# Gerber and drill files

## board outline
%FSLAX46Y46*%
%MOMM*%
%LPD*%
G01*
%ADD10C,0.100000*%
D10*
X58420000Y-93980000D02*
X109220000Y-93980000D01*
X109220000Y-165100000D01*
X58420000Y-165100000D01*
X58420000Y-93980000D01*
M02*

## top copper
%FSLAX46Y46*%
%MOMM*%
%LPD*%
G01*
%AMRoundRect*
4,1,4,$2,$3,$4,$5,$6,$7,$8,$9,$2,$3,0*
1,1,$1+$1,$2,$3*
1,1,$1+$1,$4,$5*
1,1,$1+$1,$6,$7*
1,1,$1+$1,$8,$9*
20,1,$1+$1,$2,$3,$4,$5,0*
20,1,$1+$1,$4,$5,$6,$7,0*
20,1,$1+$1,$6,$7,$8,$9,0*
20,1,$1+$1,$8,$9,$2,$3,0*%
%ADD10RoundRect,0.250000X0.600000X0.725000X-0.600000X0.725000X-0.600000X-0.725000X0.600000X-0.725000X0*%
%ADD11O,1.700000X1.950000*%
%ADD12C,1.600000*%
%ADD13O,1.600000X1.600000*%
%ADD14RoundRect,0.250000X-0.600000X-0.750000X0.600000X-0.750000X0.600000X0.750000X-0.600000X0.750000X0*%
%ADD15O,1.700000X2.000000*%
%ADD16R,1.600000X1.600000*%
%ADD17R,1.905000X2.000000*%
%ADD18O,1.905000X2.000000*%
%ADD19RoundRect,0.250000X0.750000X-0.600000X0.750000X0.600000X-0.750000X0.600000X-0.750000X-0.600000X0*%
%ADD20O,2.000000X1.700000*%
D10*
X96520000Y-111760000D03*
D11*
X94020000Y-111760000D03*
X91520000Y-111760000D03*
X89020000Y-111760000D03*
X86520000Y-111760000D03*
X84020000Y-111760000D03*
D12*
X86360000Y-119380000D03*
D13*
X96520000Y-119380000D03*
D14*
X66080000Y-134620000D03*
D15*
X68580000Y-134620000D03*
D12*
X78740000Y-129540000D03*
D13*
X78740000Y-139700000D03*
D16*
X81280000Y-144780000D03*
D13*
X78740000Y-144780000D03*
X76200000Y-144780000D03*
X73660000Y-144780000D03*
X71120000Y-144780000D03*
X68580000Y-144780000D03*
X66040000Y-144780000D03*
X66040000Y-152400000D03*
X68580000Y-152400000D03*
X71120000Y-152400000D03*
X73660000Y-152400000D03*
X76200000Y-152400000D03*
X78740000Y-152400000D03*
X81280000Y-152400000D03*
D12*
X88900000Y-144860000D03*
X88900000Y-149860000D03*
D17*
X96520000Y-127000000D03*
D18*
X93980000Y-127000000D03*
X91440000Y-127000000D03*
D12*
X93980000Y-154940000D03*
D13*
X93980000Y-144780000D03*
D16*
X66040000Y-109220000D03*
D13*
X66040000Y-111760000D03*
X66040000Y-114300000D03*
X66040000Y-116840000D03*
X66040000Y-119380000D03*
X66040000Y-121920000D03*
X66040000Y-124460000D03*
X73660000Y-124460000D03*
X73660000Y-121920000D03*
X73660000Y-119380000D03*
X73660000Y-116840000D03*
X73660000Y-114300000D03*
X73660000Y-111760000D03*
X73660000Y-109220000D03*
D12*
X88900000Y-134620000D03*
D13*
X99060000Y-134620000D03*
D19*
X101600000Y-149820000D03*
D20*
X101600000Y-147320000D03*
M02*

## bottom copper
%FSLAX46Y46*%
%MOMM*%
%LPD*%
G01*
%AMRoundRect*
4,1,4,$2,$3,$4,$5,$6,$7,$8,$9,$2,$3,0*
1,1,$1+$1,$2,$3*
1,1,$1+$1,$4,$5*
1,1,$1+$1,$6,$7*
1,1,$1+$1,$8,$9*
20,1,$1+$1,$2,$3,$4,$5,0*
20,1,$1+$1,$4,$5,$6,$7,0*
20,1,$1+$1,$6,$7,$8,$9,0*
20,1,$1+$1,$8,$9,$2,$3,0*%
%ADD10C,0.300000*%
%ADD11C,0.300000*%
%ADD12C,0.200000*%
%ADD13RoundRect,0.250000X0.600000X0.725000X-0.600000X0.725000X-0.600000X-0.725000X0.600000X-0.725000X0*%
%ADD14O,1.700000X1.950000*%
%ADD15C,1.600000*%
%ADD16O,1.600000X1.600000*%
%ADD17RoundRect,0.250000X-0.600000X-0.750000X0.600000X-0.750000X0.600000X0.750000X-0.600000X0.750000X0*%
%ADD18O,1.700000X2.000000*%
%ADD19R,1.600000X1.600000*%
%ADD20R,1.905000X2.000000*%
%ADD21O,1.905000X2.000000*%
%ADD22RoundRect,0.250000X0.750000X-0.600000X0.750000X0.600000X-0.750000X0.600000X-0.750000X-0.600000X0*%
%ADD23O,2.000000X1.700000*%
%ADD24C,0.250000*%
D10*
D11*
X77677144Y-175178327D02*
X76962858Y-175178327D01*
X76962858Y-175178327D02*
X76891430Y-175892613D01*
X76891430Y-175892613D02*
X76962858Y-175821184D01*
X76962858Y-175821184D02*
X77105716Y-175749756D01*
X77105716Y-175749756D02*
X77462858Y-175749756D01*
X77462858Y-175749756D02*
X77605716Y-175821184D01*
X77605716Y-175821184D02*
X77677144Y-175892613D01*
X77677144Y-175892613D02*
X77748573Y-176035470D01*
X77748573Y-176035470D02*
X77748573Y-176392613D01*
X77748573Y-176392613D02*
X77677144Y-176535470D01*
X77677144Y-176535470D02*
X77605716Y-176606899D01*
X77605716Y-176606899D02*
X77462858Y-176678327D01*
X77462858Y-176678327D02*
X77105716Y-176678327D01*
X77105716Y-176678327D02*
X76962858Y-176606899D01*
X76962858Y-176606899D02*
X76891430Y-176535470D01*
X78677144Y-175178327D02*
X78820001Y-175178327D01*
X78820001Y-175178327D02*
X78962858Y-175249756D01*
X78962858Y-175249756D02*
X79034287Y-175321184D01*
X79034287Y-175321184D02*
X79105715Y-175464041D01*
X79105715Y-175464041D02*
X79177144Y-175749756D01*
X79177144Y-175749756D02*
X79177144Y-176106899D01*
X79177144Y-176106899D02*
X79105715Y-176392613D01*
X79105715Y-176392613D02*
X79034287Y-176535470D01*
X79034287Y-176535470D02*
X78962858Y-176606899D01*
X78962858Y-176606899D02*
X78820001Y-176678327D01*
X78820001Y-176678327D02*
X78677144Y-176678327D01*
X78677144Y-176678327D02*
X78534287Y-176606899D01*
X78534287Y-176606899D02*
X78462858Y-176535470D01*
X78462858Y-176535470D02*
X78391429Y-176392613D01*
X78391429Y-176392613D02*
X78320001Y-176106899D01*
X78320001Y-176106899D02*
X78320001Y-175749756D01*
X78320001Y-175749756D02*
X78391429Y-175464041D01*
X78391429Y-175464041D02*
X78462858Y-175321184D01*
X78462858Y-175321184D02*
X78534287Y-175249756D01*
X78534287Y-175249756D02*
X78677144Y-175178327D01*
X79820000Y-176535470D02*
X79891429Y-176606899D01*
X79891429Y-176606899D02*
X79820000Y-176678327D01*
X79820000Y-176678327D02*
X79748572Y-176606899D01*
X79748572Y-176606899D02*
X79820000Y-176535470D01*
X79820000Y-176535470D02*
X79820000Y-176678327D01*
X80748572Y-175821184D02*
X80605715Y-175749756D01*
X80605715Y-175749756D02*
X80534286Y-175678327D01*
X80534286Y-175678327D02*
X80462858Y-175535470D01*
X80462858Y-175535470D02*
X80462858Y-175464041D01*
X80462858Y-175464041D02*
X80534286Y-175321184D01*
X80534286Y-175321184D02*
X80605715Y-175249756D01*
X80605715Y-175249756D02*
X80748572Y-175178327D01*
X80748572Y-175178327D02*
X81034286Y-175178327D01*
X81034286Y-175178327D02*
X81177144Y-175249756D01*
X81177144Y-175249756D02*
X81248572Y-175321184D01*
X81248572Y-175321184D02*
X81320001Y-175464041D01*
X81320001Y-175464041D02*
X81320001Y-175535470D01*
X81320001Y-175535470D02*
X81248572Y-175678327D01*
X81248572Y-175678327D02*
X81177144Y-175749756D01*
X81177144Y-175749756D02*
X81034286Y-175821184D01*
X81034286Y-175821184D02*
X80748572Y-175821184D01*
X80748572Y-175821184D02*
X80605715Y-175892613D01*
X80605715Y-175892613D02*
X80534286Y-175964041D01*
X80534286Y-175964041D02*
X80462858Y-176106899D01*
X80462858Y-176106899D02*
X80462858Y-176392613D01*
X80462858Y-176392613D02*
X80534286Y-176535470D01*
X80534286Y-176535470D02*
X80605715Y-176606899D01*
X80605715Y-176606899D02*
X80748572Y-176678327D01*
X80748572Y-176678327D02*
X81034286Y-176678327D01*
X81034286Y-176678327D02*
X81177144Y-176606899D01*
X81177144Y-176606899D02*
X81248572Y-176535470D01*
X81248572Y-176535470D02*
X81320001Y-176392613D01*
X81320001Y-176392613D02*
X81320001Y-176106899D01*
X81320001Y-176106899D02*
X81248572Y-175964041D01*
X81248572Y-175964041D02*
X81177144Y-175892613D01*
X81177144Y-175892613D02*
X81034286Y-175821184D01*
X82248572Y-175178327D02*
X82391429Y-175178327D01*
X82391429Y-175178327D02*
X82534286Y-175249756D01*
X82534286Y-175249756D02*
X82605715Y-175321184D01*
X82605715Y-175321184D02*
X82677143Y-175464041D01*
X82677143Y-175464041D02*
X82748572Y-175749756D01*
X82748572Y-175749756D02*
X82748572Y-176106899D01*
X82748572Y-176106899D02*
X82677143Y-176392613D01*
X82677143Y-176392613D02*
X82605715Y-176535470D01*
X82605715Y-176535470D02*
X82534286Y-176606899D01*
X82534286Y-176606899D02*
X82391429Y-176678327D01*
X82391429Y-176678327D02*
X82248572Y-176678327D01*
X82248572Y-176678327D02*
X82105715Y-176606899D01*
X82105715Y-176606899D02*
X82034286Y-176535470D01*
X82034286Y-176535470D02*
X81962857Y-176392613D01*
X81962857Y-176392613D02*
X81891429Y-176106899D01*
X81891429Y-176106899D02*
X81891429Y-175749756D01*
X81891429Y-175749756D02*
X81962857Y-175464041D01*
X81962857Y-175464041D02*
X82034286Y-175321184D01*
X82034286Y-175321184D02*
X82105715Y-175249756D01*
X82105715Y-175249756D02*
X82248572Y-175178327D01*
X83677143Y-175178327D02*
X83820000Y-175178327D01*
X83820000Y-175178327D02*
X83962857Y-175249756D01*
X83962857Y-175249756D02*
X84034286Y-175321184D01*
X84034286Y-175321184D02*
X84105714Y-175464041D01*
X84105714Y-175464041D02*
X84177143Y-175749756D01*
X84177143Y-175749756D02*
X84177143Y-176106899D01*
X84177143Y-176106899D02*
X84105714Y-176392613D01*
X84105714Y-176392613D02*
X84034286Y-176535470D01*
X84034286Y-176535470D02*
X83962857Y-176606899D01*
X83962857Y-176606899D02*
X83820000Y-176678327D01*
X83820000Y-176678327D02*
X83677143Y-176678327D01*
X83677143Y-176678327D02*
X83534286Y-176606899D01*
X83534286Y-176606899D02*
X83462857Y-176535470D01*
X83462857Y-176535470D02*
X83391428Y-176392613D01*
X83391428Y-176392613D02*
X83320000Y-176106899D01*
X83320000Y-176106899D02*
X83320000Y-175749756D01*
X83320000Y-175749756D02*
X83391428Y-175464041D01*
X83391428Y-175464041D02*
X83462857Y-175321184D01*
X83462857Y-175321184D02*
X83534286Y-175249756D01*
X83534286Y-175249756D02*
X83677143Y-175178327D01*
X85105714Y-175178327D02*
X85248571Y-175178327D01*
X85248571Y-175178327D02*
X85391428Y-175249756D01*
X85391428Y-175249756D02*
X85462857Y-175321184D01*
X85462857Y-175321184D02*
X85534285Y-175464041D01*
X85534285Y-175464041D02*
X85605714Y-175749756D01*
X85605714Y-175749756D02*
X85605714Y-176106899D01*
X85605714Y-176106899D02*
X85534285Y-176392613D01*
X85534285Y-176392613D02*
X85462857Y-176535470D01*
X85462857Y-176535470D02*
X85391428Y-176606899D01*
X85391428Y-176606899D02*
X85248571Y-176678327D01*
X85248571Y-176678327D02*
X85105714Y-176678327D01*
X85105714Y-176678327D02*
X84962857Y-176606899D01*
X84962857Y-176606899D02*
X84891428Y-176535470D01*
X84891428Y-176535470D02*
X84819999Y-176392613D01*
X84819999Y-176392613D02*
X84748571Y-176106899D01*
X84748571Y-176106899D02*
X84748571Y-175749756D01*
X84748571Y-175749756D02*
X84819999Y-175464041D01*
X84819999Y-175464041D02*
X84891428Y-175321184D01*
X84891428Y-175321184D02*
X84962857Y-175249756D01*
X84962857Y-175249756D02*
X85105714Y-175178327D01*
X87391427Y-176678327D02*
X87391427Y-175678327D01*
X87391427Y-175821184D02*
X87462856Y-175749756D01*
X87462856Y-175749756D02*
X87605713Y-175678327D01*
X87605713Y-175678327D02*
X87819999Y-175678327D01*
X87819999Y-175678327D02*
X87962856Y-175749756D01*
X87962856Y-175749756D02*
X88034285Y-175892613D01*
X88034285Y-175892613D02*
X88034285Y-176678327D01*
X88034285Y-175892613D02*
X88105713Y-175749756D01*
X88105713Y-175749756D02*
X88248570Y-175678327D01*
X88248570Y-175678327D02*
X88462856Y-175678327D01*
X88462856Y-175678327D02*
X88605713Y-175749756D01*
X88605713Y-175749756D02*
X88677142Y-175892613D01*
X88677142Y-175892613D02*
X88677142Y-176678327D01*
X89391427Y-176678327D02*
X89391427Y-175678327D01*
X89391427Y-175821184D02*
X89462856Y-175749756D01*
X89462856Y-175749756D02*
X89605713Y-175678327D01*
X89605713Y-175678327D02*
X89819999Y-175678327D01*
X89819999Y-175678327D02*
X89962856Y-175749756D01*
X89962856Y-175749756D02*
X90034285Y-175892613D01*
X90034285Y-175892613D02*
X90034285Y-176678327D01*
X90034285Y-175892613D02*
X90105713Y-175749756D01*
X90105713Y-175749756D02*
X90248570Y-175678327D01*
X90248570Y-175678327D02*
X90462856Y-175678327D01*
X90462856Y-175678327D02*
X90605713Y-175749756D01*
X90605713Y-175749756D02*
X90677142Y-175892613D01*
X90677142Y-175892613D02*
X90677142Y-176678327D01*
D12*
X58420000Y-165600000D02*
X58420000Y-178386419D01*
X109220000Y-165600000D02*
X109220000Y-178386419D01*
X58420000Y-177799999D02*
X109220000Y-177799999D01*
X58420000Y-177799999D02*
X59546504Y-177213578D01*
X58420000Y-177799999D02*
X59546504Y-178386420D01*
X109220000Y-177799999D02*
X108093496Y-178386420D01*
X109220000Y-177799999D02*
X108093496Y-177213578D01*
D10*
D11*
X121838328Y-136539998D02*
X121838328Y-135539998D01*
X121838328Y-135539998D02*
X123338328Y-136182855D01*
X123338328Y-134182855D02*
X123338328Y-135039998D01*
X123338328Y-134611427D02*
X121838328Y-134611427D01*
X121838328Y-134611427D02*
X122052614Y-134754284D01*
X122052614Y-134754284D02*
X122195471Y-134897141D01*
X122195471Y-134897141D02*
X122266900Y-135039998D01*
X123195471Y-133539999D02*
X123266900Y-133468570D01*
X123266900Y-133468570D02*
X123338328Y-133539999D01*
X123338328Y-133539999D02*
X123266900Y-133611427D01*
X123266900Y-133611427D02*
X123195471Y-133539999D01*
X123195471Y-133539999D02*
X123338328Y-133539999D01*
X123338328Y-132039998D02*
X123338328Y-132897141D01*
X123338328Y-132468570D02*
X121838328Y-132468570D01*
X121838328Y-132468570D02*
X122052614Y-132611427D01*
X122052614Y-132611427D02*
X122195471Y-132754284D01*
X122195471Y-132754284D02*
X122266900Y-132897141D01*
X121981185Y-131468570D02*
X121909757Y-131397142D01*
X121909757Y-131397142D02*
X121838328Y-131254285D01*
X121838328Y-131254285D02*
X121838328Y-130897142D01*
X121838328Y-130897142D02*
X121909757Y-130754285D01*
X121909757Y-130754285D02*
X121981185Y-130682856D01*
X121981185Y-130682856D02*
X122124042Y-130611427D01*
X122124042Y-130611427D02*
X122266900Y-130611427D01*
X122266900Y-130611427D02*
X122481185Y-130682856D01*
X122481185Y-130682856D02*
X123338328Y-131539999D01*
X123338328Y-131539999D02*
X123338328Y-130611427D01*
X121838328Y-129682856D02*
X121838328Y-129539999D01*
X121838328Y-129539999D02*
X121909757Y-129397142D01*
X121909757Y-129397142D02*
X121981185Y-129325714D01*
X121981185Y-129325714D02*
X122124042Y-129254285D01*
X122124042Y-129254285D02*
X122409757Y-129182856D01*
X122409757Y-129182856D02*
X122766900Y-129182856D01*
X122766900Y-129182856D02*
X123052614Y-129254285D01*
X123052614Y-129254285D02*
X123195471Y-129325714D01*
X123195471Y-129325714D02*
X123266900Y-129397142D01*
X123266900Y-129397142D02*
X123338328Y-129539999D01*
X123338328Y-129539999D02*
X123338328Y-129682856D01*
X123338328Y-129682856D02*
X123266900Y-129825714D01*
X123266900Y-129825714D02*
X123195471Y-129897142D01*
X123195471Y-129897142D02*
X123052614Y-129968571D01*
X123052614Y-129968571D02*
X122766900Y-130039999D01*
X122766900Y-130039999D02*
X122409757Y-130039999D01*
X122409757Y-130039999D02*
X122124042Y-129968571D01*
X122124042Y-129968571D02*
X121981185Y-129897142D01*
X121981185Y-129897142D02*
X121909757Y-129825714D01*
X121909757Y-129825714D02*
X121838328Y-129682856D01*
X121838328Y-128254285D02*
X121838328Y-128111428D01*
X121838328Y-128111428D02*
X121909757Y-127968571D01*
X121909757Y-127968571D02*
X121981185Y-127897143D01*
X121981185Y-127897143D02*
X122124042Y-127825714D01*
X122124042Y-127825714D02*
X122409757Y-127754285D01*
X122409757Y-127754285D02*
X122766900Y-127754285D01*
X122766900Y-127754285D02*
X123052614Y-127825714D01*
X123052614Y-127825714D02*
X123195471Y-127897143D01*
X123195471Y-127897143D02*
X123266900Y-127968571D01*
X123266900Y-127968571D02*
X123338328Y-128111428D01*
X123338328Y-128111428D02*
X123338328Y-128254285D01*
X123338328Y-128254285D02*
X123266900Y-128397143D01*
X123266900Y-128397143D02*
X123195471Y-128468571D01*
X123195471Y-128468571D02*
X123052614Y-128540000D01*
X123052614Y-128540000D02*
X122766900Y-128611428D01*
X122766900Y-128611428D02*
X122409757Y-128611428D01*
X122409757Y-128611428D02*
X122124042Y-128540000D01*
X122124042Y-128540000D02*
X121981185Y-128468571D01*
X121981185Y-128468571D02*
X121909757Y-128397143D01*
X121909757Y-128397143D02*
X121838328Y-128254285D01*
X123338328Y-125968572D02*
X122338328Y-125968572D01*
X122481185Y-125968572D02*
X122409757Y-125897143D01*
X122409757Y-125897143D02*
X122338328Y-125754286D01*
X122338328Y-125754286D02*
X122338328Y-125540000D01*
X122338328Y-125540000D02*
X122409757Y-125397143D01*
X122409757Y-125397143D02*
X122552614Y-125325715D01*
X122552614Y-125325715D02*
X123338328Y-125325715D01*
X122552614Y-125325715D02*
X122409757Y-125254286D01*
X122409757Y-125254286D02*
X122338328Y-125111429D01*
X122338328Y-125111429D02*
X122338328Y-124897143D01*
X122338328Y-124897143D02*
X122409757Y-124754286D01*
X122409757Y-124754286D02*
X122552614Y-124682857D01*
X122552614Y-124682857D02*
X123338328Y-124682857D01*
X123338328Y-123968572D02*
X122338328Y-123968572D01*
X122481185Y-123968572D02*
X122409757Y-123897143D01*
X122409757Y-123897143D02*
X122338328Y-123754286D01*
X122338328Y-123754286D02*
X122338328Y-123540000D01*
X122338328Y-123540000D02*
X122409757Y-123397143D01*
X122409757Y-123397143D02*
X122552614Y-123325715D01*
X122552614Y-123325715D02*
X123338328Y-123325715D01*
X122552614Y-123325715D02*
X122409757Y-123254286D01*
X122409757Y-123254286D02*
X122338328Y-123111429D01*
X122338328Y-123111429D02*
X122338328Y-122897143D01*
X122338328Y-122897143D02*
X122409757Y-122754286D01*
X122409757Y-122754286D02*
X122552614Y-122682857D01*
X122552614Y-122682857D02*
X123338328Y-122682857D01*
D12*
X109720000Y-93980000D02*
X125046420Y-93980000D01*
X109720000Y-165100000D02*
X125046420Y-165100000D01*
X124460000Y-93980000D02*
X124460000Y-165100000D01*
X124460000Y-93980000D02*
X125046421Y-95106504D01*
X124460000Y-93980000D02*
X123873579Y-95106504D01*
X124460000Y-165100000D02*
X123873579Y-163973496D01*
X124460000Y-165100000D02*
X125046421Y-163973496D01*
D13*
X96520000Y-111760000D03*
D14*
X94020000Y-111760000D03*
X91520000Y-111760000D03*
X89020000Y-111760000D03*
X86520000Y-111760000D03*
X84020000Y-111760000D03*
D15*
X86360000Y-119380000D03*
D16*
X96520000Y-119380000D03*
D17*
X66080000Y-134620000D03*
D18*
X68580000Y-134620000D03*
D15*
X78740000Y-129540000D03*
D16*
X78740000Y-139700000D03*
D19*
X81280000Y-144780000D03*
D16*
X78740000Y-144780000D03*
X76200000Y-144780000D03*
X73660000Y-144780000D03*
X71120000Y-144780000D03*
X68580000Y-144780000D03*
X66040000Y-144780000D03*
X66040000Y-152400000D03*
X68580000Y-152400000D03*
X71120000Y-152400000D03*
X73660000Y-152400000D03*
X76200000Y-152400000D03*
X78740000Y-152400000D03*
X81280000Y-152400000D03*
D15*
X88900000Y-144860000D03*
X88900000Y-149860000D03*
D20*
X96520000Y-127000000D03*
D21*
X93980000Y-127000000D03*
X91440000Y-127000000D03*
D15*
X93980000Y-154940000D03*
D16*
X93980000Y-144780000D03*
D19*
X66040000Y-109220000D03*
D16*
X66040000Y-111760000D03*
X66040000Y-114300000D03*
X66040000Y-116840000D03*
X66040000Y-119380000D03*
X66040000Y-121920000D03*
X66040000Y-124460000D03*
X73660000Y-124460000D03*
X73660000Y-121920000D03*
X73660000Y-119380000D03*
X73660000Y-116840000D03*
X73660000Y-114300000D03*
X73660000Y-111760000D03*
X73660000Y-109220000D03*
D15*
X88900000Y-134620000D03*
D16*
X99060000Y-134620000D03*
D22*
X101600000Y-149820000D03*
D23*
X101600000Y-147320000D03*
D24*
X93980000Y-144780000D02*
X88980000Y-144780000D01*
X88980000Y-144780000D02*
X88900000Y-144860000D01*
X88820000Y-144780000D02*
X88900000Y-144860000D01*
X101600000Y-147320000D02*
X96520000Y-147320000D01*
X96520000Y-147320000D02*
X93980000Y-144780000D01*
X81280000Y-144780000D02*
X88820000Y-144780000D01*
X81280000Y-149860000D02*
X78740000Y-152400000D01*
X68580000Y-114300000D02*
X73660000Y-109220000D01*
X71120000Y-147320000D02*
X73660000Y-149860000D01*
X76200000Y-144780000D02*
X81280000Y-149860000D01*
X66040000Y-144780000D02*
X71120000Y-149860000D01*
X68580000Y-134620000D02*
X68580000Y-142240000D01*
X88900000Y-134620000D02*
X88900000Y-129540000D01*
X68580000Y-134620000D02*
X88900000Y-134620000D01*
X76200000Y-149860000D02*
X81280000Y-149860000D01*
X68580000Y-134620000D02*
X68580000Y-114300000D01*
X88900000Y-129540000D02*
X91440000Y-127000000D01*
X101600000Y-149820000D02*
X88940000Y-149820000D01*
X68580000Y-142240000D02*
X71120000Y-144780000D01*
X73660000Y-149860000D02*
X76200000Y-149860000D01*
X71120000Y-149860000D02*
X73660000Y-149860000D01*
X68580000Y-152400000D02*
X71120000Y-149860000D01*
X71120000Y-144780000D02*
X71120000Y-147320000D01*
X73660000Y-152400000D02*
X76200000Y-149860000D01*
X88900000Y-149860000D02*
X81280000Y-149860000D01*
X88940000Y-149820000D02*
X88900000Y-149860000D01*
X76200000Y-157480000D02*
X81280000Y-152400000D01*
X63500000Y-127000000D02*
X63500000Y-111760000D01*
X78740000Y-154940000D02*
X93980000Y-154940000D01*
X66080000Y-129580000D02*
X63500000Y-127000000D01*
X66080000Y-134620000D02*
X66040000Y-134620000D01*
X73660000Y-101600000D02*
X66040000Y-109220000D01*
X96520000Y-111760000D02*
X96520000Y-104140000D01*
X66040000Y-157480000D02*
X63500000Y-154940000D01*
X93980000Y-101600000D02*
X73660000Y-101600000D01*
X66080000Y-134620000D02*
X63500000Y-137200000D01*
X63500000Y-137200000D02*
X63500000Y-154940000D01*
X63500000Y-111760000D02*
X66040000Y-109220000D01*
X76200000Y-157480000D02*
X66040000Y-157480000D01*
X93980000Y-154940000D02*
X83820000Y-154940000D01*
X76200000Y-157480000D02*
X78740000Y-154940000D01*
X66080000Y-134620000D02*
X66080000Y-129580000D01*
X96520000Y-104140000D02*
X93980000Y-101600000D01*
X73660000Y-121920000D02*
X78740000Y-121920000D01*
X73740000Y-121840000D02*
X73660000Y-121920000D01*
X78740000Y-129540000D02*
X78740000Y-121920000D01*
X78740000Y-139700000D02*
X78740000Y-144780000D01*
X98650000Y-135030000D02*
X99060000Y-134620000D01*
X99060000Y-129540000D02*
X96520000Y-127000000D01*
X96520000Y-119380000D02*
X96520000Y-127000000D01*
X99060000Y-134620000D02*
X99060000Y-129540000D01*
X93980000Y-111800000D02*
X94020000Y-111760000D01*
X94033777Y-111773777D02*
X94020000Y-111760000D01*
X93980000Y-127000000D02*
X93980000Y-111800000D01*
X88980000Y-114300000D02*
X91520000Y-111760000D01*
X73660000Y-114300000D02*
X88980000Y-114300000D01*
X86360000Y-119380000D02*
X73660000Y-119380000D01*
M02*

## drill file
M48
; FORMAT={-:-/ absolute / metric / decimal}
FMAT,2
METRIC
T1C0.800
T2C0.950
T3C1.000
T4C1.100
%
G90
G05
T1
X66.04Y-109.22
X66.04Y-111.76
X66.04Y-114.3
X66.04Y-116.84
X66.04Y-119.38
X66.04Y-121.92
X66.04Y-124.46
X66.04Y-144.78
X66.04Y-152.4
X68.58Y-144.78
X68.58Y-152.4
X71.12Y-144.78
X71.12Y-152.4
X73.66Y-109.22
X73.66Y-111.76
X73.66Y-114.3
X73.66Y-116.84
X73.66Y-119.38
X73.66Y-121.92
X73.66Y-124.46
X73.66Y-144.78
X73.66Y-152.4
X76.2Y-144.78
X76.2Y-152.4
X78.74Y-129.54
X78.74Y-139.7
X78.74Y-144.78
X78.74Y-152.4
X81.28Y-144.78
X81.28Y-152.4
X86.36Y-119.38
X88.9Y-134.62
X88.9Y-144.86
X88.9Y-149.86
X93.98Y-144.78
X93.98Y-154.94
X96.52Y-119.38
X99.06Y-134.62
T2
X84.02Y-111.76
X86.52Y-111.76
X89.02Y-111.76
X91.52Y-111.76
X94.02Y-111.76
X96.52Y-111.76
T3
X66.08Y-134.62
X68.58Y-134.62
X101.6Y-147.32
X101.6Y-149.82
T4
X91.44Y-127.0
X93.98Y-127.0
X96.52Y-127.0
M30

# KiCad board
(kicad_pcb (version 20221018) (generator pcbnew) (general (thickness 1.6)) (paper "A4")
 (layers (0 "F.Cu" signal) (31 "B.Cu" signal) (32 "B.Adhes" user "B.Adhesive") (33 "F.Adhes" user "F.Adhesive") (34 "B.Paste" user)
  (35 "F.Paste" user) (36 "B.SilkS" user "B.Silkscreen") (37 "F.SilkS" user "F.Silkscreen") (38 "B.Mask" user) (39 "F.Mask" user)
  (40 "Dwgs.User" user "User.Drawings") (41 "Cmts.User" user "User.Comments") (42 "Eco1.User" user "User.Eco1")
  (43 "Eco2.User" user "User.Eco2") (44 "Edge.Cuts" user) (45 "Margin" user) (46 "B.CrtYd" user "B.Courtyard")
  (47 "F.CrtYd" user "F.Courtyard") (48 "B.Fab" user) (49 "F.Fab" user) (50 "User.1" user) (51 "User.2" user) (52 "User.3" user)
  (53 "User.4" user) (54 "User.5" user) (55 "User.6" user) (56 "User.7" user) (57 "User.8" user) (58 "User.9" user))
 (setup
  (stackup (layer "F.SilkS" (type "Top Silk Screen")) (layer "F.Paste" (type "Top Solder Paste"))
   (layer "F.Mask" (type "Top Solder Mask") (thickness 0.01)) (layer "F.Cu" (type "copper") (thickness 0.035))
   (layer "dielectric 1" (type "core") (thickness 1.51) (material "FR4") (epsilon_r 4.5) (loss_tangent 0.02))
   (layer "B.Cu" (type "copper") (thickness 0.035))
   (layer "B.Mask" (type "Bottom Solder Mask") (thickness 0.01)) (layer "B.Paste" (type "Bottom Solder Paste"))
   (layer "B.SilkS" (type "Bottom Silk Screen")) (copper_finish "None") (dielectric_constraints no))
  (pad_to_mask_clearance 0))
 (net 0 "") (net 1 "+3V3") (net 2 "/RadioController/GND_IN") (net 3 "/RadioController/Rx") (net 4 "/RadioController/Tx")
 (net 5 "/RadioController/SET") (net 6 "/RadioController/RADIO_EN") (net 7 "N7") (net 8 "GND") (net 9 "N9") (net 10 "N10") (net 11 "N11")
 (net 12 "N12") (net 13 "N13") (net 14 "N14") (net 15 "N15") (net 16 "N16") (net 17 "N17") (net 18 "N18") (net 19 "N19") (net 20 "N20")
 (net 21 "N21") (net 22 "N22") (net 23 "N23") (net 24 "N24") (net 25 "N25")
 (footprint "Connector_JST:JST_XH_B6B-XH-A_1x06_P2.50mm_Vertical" (layer "F.Cu") (at 96.52 111.76 180)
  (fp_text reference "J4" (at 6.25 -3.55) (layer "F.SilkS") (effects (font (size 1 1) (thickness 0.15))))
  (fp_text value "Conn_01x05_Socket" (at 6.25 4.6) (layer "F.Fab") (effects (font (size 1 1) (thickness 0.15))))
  (pad "1" thru_hole roundrect (at 0 0 180) (size 1.7 1.95) (drill 0.95) (layers "*.Cu" "*.Mask") (roundrect_rratio 0.1470588235)
   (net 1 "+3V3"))
  (pad "2" thru_hole oval (at 2.5 0 180) (size 1.7 1.95) (drill 0.95) (layers "*.Cu" "*.Mask") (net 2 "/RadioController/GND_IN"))
  (pad "3" thru_hole oval (at 5 0 180) (size 1.7 1.95) (drill 0.95) (layers "*.Cu" "*.Mask") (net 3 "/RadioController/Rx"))
  (pad "4" thru_hole oval (at 7.5 0 180) (size 1.7 1.95) (drill 0.95) (layers "*.Cu" "*.Mask") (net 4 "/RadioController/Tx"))
  (pad "5" thru_hole oval (at 10 0 180) (size 1.7 1.95) (drill 0.95) (layers "*.Cu" "*.Mask") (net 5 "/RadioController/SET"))
  (pad "6" thru_hole oval (at 12.5 0 180) (size 1.7 1.95) (drill 0.95) (layers "*.Cu" "*.Mask")))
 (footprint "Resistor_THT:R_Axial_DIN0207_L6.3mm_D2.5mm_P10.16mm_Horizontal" (layer "F.Cu") (at 86.36 119.38)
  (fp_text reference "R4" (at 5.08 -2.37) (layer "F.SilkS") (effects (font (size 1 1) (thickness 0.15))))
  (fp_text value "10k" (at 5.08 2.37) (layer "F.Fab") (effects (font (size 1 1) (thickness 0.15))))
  (pad "1" thru_hole circle (at 0 0) (size 1.6 1.6) (drill 0.8) (layers "*.Cu" "*.Mask") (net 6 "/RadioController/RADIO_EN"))
  (pad "2" thru_hole oval (at 10.16 0) (size 1.6 1.6) (drill 0.8) (layers "*.Cu" "*.Mask") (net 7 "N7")))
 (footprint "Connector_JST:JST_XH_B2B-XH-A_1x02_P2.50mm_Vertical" (layer "F.Cu") (at 66.08 134.62)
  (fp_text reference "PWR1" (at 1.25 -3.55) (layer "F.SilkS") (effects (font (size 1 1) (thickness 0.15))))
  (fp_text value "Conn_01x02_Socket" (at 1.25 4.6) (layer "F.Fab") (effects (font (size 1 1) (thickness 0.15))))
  (pad "1" thru_hole roundrect (at 0 0) (size 1.7 2) (drill 1) (layers "*.Cu" "*.Mask") (roundrect_rratio 0.1470588235) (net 1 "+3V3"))
  (pad "2" thru_hole oval (at 2.5 0) (size 1.7 2) (drill 1) (layers "*.Cu" "*.Mask") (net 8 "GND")))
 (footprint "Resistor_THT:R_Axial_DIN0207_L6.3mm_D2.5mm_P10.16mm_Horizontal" (layer "F.Cu") (at 78.74 129.54 -90)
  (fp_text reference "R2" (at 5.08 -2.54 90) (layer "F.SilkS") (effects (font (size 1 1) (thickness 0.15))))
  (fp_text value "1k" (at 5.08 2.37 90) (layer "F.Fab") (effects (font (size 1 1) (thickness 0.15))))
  (pad "1" thru_hole circle (at 0 0 270) (size 1.6 1.6) (drill 0.8) (layers "*.Cu" "*.Mask") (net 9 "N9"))
  (pad "2" thru_hole oval (at 10.16 0 270) (size 1.6 1.6) (drill 0.8) (layers "*.Cu" "*.Mask") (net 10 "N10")))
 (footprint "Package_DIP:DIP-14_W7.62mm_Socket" (layer "F.Cu") (at 81.28 144.78 -90)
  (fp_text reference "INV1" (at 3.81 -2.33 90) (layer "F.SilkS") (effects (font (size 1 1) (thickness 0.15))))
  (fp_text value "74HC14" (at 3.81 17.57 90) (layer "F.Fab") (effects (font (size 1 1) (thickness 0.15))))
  (pad "1" thru_hole rect (at 0 0 270) (size 1.6 1.6) (drill 0.8) (layers "*.Cu" "*.Mask") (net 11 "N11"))
  (pad "2" thru_hole oval (at 0 2.54 270) (size 1.6 1.6) (drill 0.8) (layers "*.Cu" "*.Mask") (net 10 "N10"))
  (pad "3" thru_hole oval (at 0 5.08 270) (size 1.6 1.6) (drill 0.8) (layers "*.Cu" "*.Mask") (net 8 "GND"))
  (pad "4" thru_hole oval (at 0 7.62 270) (size 1.6 1.6) (drill 0.8) (layers "*.Cu" "*.Mask") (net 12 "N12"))
  (pad "5" thru_hole oval (at 0 10.16 270) (size 1.6 1.6) (drill 0.8) (layers "*.Cu" "*.Mask") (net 8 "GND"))
  (pad "6" thru_hole oval (at 0 12.7 270) (size 1.6 1.6) (drill 0.8) (layers "*.Cu" "*.Mask") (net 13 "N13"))
  (pad "7" thru_hole oval (at 0 15.24 270) (size 1.6 1.6) (drill 0.8) (layers "*.Cu" "*.Mask") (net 8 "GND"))
  (pad "8" thru_hole oval (at 7.62 15.24 270) (size 1.6 1.6) (drill 0.8) (layers "*.Cu" "*.Mask") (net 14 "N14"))
  (pad "9" thru_hole oval (at 7.62 12.7 270) (size 1.6 1.6) (drill 0.8) (layers "*.Cu" "*.Mask") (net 8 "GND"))
  (pad "10" thru_hole oval (at 7.62 10.16 270) (size 1.6 1.6) (drill 0.8) (layers "*.Cu" "*.Mask") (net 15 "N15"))
  (pad "11" thru_hole oval (at 7.62 7.62 270) (size 1.6 1.6) (drill 0.8) (layers "*.Cu" "*.Mask") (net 8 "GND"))
  (pad "12" thru_hole oval (at 7.62 5.08 270) (size 1.6 1.6) (drill 0.8) (layers "*.Cu" "*.Mask") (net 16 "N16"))
  (pad "13" thru_hole oval (at 7.62 2.54 270) (size 1.6 1.6) (drill 0.8) (layers "*.Cu" "*.Mask") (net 8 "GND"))
  (pad "14" thru_hole oval (at 7.62 0 270) (size 1.6 1.6) (drill 0.8) (layers "*.Cu" "*.Mask") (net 1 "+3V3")))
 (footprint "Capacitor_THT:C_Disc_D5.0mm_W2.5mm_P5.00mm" (layer "F.Cu") (at 88.9 144.86 -90)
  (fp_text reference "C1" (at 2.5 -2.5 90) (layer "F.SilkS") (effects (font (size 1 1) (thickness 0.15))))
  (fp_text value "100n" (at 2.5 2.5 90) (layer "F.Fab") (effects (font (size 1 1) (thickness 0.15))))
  (pad "1" thru_hole circle (at 0 0 270) (size 1.6 1.6) (drill 0.8) (layers "*.Cu" "*.Mask") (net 11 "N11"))
  (pad "2" thru_hole circle (at 5 0 270) (size 1.6 1.6) (drill 0.8) (layers "*.Cu" "*.Mask") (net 8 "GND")))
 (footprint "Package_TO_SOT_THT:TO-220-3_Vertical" (layer "F.Cu") (at 96.52 127 180)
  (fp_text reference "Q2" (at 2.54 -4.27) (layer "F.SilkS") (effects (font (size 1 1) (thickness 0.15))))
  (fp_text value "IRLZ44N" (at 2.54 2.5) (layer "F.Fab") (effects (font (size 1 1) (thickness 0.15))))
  (pad "1" thru_hole rect (at 0 0 180) (size 1.905 2) (drill 1.1) (layers "*.Cu" "*.Mask") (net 7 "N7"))
  (pad "2" thru_hole oval (at 2.54 0 180) (size 1.905 2) (drill 1.1) (layers "*.Cu" "*.Mask") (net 2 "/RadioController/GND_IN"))
  (pad "3" thru_hole oval (at 5.08 0 180) (size 1.905 2) (drill 1.1) (layers "*.Cu" "*.Mask") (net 8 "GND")))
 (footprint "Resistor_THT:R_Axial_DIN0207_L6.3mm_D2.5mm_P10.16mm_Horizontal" (layer "F.Cu") (at 93.98 154.94 90)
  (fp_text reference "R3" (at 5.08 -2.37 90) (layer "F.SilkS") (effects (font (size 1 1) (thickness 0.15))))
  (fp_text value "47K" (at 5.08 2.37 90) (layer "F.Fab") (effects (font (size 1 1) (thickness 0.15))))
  (pad "1" thru_hole circle (at 0 0 90) (size 1.6 1.6) (drill 0.8) (layers "*.Cu" "*.Mask") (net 1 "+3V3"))
  (pad "2" thru_hole oval (at 10.16 0 90) (size 1.6 1.6) (drill 0.8) (layers "*.Cu" "*.Mask") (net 11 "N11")))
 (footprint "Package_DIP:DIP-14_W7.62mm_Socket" (layer "F.Cu") (at 66.04 109.22)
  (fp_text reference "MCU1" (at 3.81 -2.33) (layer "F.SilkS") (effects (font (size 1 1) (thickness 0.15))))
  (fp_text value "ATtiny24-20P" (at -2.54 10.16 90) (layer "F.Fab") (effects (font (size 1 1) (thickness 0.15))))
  (pad "1" thru_hole rect (at 0 0) (size 1.6 1.6) (drill 0.8) (layers "*.Cu" "*.Mask") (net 1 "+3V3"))
  (pad "2" thru_hole oval (at 0 2.54) (size 1.6 1.6) (drill 0.8) (layers "*.Cu" "*.Mask") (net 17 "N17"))
  (pad "3" thru_hole oval (at 0 5.08) (size 1.6 1.6) (drill 0.8) (layers "*.Cu" "*.Mask") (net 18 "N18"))
  (pad "4" thru_hole oval (at 0 7.62) (size 1.6 1.6) (drill 0.8) (layers "*.Cu" "*.Mask") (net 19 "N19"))
  (pad "5" thru_hole oval (at 0 10.16) (size 1.6 1.6) (drill 0.8) (layers "*.Cu" "*.Mask") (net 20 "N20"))
  (pad "6" thru_hole oval (at 0 12.7) (size 1.6 1.6) (drill 0.8) (layers "*.Cu" "*.Mask") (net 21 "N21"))
  (pad "7" thru_hole oval (at 0 15.24) (size 1.6 1.6) (drill 0.8) (layers "*.Cu" "*.Mask") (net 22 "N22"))
  (pad "8" thru_hole oval (at 7.62 15.24) (size 1.6 1.6) (drill 0.8) (layers "*.Cu" "*.Mask") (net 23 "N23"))
  (pad "9" thru_hole oval (at 7.62 12.7) (size 1.6 1.6) (drill 0.8) (layers "*.Cu" "*.Mask") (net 9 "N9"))
  (pad "10" thru_hole oval (at 7.62 10.16) (size 1.6 1.6) (drill 0.8) (layers "*.Cu" "*.Mask") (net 6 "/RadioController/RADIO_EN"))
  (pad "11" thru_hole oval (at 7.62 7.62) (size 1.6 1.6) (drill 0.8) (layers "*.Cu" "*.Mask") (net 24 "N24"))
  (pad "12" thru_hole oval (at 7.62 5.08) (size 1.6 1.6) (drill 0.8) (layers "*.Cu" "*.Mask") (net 3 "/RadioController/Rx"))
  (pad "13" thru_hole oval (at 7.62 2.54) (size 1.6 1.6) (drill 0.8) (layers "*.Cu" "*.Mask") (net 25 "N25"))
  (pad "14" thru_hole oval (at 7.62 0) (size 1.6 1.6) (drill 0.8) (layers "*.Cu" "*.Mask") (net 8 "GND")))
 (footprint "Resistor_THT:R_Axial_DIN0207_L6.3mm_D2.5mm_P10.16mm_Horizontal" (layer "F.Cu") (at 88.9 134.62)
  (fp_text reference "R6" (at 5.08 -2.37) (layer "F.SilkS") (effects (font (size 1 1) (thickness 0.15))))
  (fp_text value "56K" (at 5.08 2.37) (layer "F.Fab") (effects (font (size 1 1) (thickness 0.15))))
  (pad "1" thru_hole circle (at 0 0) (size 1.6 1.6) (drill 0.8) (layers "*.Cu" "*.Mask") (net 8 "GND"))
  (pad "2" thru_hole oval (at 10.16 0) (size 1.6 1.6) (drill 0.8) (layers "*.Cu" "*.Mask") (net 7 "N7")))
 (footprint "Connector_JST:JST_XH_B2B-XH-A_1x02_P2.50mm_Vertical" (layer "F.Cu") (at 101.6 149.82 90)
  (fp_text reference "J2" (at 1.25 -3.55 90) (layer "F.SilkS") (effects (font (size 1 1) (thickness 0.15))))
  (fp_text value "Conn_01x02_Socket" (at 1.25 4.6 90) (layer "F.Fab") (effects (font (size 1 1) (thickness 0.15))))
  (pad "1" thru_hole roundrect (at 0 0 90) (size 1.7 2) (drill 1) (layers "*.Cu" "*.Mask") (roundrect_rratio 0.1470588235) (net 8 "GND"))
  (pad "2" thru_hole oval (at 2.5 0 90) (size 1.7 2) (drill 1) (layers "*.Cu" "*.Mask") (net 11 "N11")))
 (gr_rect (start 58.42 93.98) (end 109.22 165.1) (stroke (width 0.1) (type default)) (fill none) (layer "Edge.Cuts"))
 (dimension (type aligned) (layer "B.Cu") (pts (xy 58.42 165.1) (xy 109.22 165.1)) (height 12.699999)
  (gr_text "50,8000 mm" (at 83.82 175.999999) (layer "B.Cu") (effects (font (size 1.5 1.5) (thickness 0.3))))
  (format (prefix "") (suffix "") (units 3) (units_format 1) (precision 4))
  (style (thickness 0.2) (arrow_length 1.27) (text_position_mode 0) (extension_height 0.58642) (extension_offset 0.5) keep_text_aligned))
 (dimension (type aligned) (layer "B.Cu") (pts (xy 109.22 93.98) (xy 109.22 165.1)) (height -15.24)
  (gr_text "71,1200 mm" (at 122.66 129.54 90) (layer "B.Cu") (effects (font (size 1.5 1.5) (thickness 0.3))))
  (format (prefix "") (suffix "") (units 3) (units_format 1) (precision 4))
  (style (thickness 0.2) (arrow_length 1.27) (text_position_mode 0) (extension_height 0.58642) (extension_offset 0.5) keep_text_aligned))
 (segment (start 93.98 144.78) (end 88.98 144.78) (width 0.25) (layer "B.Cu") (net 11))
 (segment (start 88.98 144.78) (end 88.9 144.86) (width 0.25) (layer "B.Cu") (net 11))
 (segment (start 88.82 144.78) (end 88.9 144.86) (width 0.25) (layer "B.Cu") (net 11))
 (segment (start 101.6 147.32) (end 96.52 147.32) (width 0.25) (layer "B.Cu") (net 11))
 (segment (start 96.52 147.32) (end 93.98 144.78) (width 0.25) (layer "B.Cu") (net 11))
 (segment (start 81.28 144.78) (end 88.82 144.78) (width 0.25) (layer "B.Cu") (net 11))
 (segment (start 81.28 149.86) (end 78.74 152.4) (width 0.25) (layer "B.Cu") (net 8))
 (segment (start 68.58 114.3) (end 73.66 109.22) (width 0.25) (layer "B.Cu") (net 8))
 (segment (start 71.12 147.32) (end 73.66 149.86) (width 0.25) (layer "B.Cu") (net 8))
 (segment (start 76.2 144.78) (end 81.28 149.86) (width 0.25) (layer "B.Cu") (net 8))
 (segment (start 66.04 144.78) (end 71.12 149.86) (width 0.25) (layer "B.Cu") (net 8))
 (segment (start 68.58 134.62) (end 68.58 142.24) (width 0.25) (layer "B.Cu") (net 8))
 (segment (start 88.9 134.62) (end 88.9 129.54) (width 0.25) (layer "B.Cu") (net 8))
 (segment (start 68.58 134.62) (end 88.9 134.62) (width 0.25) (layer "B.Cu") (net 8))
 (segment (start 76.2 149.86) (end 81.28 149.86) (width 0.25) (layer "B.Cu") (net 8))
 (segment (start 68.58 134.62) (end 68.58 114.3) (width 0.25) (layer "B.Cu") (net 8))
 (segment (start 88.9 129.54) (end 91.44 127) (width 0.25) (layer "B.Cu") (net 8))
 (segment (start 101.6 149.82) (end 88.94 149.82) (width 0.25) (layer "B.Cu") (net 8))
 (segment (start 68.58 142.24) (end 71.12 144.78) (width 0.25) (layer "B.Cu") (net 8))
 (segment (start 73.66 149.86) (end 76.2 149.86) (width 0.25) (layer "B.Cu") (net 8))
 (segment (start 71.12 149.86) (end 73.66 149.86) (width 0.25) (layer "B.Cu") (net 8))
 (segment (start 68.58 152.4) (end 71.12 149.86) (width 0.25) (layer "B.Cu") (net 8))
 (segment (start 71.12 144.78) (end 71.12 147.32) (width 0.25) (layer "B.Cu") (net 8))
 (segment (start 73.66 152.4) (end 76.2 149.86) (width 0.25) (layer "B.Cu") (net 8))
 (segment (start 88.9 149.86) (end 81.28 149.86) (width 0.25) (layer "B.Cu") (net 8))
 (segment (start 88.94 149.82) (end 88.9 149.86) (width 0.25) (layer "B.Cu") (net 8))
 (segment (start 76.2 157.48) (end 81.28 152.4) (width 0.25) (layer "B.Cu") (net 1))
 (segment (start 63.5 127) (end 63.5 111.76) (width 0.25) (layer "B.Cu") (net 1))
 (segment (start 78.74 154.94) (end 93.98 154.94) (width 0.25) (layer "B.Cu") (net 1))
 (segment (start 66.08 129.58) (end 63.5 127) (width 0.25) (layer "B.Cu") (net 1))
 (segment (start 66.08 134.62) (end 66.04 134.62) (width 0.25) (layer "B.Cu") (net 1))
 (segment (start 73.66 101.6) (end 66.04 109.22) (width 0.25) (layer "B.Cu") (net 1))
 (segment (start 96.52 111.76) (end 96.52 104.14) (width 0.25) (layer "B.Cu") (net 1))
 (segment (start 66.04 157.48) (end 63.5 154.94) (width 0.25) (layer "B.Cu") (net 1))
 (segment (start 93.98 101.6) (end 73.66 101.6) (width 0.25) (layer "B.Cu") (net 1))
 (segment (start 66.08 134.62) (end 63.5 137.2) (width 0.25) (layer "B.Cu") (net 1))
 (segment (start 63.5 137.2) (end 63.5 154.94) (width 0.25) (layer "B.Cu") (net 1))
 (segment (start 63.5 111.76) (end 66.04 109.22) (width 0.25) (layer "B.Cu") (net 1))
 (segment (start 76.2 157.48) (end 66.04 157.48) (width 0.25) (layer "B.Cu") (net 1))
 (segment (start 93.98 154.94) (end 83.82 154.94) (width 0.25) (layer "B.Cu") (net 1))
 (segment (start 76.2 157.48) (end 78.74 154.94) (width 0.25) (layer "B.Cu") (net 1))
 (segment (start 66.08 134.62) (end 66.08 129.58) (width 0.25) (layer "B.Cu") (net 1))
 (segment (start 96.52 104.14) (end 93.98 101.6) (width 0.25) (layer "B.Cu") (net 1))
 (segment (start 73.66 121.92) (end 78.74 121.92) (width 0.25) (layer "B.Cu") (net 9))
 (segment (start 73.74 121.84) (end 73.66 121.92) (width 0.25) (layer "B.Cu") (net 9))
 (segment (start 78.74 129.54) (end 78.74 121.92) (width 0.25) (layer "B.Cu") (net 9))
 (segment (start 78.74 139.7) (end 78.74 144.78) (width 0.25) (layer "B.Cu") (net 10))
 (segment (start 98.65 135.03) (end 99.06 134.62) (width 0.25) (layer "B.Cu") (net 7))
 (segment (start 99.06 129.54) (end 96.52 127) (width 0.25) (layer "B.Cu") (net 7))
 (segment (start 96.52 119.38) (end 96.52 127) (width 0.25) (layer "B.Cu") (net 7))
 (segment (start 99.06 134.62) (end 99.06 129.54) (width 0.25) (layer "B.Cu") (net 7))
 (segment (start 93.98 111.8) (end 94.02 111.76) (width 0.25) (layer "B.Cu") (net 2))
 (segment (start 94.033777 111.773777) (end 94.02 111.76) (width 0.25) (layer "B.Cu") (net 2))
 (segment (start 93.98 127) (end 93.98 111.8) (width 0.25) (layer "B.Cu") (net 2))
 (segment (start 88.98 114.3) (end 91.52 111.76) (width 0.25) (layer "B.Cu") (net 3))
 (segment (start 73.66 114.3) (end 88.98 114.3) (width 0.25) (layer "B.Cu") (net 3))
 (segment (start 86.36 119.38) (end 73.66 119.38) (width 0.25) (layer "B.Cu") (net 6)))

